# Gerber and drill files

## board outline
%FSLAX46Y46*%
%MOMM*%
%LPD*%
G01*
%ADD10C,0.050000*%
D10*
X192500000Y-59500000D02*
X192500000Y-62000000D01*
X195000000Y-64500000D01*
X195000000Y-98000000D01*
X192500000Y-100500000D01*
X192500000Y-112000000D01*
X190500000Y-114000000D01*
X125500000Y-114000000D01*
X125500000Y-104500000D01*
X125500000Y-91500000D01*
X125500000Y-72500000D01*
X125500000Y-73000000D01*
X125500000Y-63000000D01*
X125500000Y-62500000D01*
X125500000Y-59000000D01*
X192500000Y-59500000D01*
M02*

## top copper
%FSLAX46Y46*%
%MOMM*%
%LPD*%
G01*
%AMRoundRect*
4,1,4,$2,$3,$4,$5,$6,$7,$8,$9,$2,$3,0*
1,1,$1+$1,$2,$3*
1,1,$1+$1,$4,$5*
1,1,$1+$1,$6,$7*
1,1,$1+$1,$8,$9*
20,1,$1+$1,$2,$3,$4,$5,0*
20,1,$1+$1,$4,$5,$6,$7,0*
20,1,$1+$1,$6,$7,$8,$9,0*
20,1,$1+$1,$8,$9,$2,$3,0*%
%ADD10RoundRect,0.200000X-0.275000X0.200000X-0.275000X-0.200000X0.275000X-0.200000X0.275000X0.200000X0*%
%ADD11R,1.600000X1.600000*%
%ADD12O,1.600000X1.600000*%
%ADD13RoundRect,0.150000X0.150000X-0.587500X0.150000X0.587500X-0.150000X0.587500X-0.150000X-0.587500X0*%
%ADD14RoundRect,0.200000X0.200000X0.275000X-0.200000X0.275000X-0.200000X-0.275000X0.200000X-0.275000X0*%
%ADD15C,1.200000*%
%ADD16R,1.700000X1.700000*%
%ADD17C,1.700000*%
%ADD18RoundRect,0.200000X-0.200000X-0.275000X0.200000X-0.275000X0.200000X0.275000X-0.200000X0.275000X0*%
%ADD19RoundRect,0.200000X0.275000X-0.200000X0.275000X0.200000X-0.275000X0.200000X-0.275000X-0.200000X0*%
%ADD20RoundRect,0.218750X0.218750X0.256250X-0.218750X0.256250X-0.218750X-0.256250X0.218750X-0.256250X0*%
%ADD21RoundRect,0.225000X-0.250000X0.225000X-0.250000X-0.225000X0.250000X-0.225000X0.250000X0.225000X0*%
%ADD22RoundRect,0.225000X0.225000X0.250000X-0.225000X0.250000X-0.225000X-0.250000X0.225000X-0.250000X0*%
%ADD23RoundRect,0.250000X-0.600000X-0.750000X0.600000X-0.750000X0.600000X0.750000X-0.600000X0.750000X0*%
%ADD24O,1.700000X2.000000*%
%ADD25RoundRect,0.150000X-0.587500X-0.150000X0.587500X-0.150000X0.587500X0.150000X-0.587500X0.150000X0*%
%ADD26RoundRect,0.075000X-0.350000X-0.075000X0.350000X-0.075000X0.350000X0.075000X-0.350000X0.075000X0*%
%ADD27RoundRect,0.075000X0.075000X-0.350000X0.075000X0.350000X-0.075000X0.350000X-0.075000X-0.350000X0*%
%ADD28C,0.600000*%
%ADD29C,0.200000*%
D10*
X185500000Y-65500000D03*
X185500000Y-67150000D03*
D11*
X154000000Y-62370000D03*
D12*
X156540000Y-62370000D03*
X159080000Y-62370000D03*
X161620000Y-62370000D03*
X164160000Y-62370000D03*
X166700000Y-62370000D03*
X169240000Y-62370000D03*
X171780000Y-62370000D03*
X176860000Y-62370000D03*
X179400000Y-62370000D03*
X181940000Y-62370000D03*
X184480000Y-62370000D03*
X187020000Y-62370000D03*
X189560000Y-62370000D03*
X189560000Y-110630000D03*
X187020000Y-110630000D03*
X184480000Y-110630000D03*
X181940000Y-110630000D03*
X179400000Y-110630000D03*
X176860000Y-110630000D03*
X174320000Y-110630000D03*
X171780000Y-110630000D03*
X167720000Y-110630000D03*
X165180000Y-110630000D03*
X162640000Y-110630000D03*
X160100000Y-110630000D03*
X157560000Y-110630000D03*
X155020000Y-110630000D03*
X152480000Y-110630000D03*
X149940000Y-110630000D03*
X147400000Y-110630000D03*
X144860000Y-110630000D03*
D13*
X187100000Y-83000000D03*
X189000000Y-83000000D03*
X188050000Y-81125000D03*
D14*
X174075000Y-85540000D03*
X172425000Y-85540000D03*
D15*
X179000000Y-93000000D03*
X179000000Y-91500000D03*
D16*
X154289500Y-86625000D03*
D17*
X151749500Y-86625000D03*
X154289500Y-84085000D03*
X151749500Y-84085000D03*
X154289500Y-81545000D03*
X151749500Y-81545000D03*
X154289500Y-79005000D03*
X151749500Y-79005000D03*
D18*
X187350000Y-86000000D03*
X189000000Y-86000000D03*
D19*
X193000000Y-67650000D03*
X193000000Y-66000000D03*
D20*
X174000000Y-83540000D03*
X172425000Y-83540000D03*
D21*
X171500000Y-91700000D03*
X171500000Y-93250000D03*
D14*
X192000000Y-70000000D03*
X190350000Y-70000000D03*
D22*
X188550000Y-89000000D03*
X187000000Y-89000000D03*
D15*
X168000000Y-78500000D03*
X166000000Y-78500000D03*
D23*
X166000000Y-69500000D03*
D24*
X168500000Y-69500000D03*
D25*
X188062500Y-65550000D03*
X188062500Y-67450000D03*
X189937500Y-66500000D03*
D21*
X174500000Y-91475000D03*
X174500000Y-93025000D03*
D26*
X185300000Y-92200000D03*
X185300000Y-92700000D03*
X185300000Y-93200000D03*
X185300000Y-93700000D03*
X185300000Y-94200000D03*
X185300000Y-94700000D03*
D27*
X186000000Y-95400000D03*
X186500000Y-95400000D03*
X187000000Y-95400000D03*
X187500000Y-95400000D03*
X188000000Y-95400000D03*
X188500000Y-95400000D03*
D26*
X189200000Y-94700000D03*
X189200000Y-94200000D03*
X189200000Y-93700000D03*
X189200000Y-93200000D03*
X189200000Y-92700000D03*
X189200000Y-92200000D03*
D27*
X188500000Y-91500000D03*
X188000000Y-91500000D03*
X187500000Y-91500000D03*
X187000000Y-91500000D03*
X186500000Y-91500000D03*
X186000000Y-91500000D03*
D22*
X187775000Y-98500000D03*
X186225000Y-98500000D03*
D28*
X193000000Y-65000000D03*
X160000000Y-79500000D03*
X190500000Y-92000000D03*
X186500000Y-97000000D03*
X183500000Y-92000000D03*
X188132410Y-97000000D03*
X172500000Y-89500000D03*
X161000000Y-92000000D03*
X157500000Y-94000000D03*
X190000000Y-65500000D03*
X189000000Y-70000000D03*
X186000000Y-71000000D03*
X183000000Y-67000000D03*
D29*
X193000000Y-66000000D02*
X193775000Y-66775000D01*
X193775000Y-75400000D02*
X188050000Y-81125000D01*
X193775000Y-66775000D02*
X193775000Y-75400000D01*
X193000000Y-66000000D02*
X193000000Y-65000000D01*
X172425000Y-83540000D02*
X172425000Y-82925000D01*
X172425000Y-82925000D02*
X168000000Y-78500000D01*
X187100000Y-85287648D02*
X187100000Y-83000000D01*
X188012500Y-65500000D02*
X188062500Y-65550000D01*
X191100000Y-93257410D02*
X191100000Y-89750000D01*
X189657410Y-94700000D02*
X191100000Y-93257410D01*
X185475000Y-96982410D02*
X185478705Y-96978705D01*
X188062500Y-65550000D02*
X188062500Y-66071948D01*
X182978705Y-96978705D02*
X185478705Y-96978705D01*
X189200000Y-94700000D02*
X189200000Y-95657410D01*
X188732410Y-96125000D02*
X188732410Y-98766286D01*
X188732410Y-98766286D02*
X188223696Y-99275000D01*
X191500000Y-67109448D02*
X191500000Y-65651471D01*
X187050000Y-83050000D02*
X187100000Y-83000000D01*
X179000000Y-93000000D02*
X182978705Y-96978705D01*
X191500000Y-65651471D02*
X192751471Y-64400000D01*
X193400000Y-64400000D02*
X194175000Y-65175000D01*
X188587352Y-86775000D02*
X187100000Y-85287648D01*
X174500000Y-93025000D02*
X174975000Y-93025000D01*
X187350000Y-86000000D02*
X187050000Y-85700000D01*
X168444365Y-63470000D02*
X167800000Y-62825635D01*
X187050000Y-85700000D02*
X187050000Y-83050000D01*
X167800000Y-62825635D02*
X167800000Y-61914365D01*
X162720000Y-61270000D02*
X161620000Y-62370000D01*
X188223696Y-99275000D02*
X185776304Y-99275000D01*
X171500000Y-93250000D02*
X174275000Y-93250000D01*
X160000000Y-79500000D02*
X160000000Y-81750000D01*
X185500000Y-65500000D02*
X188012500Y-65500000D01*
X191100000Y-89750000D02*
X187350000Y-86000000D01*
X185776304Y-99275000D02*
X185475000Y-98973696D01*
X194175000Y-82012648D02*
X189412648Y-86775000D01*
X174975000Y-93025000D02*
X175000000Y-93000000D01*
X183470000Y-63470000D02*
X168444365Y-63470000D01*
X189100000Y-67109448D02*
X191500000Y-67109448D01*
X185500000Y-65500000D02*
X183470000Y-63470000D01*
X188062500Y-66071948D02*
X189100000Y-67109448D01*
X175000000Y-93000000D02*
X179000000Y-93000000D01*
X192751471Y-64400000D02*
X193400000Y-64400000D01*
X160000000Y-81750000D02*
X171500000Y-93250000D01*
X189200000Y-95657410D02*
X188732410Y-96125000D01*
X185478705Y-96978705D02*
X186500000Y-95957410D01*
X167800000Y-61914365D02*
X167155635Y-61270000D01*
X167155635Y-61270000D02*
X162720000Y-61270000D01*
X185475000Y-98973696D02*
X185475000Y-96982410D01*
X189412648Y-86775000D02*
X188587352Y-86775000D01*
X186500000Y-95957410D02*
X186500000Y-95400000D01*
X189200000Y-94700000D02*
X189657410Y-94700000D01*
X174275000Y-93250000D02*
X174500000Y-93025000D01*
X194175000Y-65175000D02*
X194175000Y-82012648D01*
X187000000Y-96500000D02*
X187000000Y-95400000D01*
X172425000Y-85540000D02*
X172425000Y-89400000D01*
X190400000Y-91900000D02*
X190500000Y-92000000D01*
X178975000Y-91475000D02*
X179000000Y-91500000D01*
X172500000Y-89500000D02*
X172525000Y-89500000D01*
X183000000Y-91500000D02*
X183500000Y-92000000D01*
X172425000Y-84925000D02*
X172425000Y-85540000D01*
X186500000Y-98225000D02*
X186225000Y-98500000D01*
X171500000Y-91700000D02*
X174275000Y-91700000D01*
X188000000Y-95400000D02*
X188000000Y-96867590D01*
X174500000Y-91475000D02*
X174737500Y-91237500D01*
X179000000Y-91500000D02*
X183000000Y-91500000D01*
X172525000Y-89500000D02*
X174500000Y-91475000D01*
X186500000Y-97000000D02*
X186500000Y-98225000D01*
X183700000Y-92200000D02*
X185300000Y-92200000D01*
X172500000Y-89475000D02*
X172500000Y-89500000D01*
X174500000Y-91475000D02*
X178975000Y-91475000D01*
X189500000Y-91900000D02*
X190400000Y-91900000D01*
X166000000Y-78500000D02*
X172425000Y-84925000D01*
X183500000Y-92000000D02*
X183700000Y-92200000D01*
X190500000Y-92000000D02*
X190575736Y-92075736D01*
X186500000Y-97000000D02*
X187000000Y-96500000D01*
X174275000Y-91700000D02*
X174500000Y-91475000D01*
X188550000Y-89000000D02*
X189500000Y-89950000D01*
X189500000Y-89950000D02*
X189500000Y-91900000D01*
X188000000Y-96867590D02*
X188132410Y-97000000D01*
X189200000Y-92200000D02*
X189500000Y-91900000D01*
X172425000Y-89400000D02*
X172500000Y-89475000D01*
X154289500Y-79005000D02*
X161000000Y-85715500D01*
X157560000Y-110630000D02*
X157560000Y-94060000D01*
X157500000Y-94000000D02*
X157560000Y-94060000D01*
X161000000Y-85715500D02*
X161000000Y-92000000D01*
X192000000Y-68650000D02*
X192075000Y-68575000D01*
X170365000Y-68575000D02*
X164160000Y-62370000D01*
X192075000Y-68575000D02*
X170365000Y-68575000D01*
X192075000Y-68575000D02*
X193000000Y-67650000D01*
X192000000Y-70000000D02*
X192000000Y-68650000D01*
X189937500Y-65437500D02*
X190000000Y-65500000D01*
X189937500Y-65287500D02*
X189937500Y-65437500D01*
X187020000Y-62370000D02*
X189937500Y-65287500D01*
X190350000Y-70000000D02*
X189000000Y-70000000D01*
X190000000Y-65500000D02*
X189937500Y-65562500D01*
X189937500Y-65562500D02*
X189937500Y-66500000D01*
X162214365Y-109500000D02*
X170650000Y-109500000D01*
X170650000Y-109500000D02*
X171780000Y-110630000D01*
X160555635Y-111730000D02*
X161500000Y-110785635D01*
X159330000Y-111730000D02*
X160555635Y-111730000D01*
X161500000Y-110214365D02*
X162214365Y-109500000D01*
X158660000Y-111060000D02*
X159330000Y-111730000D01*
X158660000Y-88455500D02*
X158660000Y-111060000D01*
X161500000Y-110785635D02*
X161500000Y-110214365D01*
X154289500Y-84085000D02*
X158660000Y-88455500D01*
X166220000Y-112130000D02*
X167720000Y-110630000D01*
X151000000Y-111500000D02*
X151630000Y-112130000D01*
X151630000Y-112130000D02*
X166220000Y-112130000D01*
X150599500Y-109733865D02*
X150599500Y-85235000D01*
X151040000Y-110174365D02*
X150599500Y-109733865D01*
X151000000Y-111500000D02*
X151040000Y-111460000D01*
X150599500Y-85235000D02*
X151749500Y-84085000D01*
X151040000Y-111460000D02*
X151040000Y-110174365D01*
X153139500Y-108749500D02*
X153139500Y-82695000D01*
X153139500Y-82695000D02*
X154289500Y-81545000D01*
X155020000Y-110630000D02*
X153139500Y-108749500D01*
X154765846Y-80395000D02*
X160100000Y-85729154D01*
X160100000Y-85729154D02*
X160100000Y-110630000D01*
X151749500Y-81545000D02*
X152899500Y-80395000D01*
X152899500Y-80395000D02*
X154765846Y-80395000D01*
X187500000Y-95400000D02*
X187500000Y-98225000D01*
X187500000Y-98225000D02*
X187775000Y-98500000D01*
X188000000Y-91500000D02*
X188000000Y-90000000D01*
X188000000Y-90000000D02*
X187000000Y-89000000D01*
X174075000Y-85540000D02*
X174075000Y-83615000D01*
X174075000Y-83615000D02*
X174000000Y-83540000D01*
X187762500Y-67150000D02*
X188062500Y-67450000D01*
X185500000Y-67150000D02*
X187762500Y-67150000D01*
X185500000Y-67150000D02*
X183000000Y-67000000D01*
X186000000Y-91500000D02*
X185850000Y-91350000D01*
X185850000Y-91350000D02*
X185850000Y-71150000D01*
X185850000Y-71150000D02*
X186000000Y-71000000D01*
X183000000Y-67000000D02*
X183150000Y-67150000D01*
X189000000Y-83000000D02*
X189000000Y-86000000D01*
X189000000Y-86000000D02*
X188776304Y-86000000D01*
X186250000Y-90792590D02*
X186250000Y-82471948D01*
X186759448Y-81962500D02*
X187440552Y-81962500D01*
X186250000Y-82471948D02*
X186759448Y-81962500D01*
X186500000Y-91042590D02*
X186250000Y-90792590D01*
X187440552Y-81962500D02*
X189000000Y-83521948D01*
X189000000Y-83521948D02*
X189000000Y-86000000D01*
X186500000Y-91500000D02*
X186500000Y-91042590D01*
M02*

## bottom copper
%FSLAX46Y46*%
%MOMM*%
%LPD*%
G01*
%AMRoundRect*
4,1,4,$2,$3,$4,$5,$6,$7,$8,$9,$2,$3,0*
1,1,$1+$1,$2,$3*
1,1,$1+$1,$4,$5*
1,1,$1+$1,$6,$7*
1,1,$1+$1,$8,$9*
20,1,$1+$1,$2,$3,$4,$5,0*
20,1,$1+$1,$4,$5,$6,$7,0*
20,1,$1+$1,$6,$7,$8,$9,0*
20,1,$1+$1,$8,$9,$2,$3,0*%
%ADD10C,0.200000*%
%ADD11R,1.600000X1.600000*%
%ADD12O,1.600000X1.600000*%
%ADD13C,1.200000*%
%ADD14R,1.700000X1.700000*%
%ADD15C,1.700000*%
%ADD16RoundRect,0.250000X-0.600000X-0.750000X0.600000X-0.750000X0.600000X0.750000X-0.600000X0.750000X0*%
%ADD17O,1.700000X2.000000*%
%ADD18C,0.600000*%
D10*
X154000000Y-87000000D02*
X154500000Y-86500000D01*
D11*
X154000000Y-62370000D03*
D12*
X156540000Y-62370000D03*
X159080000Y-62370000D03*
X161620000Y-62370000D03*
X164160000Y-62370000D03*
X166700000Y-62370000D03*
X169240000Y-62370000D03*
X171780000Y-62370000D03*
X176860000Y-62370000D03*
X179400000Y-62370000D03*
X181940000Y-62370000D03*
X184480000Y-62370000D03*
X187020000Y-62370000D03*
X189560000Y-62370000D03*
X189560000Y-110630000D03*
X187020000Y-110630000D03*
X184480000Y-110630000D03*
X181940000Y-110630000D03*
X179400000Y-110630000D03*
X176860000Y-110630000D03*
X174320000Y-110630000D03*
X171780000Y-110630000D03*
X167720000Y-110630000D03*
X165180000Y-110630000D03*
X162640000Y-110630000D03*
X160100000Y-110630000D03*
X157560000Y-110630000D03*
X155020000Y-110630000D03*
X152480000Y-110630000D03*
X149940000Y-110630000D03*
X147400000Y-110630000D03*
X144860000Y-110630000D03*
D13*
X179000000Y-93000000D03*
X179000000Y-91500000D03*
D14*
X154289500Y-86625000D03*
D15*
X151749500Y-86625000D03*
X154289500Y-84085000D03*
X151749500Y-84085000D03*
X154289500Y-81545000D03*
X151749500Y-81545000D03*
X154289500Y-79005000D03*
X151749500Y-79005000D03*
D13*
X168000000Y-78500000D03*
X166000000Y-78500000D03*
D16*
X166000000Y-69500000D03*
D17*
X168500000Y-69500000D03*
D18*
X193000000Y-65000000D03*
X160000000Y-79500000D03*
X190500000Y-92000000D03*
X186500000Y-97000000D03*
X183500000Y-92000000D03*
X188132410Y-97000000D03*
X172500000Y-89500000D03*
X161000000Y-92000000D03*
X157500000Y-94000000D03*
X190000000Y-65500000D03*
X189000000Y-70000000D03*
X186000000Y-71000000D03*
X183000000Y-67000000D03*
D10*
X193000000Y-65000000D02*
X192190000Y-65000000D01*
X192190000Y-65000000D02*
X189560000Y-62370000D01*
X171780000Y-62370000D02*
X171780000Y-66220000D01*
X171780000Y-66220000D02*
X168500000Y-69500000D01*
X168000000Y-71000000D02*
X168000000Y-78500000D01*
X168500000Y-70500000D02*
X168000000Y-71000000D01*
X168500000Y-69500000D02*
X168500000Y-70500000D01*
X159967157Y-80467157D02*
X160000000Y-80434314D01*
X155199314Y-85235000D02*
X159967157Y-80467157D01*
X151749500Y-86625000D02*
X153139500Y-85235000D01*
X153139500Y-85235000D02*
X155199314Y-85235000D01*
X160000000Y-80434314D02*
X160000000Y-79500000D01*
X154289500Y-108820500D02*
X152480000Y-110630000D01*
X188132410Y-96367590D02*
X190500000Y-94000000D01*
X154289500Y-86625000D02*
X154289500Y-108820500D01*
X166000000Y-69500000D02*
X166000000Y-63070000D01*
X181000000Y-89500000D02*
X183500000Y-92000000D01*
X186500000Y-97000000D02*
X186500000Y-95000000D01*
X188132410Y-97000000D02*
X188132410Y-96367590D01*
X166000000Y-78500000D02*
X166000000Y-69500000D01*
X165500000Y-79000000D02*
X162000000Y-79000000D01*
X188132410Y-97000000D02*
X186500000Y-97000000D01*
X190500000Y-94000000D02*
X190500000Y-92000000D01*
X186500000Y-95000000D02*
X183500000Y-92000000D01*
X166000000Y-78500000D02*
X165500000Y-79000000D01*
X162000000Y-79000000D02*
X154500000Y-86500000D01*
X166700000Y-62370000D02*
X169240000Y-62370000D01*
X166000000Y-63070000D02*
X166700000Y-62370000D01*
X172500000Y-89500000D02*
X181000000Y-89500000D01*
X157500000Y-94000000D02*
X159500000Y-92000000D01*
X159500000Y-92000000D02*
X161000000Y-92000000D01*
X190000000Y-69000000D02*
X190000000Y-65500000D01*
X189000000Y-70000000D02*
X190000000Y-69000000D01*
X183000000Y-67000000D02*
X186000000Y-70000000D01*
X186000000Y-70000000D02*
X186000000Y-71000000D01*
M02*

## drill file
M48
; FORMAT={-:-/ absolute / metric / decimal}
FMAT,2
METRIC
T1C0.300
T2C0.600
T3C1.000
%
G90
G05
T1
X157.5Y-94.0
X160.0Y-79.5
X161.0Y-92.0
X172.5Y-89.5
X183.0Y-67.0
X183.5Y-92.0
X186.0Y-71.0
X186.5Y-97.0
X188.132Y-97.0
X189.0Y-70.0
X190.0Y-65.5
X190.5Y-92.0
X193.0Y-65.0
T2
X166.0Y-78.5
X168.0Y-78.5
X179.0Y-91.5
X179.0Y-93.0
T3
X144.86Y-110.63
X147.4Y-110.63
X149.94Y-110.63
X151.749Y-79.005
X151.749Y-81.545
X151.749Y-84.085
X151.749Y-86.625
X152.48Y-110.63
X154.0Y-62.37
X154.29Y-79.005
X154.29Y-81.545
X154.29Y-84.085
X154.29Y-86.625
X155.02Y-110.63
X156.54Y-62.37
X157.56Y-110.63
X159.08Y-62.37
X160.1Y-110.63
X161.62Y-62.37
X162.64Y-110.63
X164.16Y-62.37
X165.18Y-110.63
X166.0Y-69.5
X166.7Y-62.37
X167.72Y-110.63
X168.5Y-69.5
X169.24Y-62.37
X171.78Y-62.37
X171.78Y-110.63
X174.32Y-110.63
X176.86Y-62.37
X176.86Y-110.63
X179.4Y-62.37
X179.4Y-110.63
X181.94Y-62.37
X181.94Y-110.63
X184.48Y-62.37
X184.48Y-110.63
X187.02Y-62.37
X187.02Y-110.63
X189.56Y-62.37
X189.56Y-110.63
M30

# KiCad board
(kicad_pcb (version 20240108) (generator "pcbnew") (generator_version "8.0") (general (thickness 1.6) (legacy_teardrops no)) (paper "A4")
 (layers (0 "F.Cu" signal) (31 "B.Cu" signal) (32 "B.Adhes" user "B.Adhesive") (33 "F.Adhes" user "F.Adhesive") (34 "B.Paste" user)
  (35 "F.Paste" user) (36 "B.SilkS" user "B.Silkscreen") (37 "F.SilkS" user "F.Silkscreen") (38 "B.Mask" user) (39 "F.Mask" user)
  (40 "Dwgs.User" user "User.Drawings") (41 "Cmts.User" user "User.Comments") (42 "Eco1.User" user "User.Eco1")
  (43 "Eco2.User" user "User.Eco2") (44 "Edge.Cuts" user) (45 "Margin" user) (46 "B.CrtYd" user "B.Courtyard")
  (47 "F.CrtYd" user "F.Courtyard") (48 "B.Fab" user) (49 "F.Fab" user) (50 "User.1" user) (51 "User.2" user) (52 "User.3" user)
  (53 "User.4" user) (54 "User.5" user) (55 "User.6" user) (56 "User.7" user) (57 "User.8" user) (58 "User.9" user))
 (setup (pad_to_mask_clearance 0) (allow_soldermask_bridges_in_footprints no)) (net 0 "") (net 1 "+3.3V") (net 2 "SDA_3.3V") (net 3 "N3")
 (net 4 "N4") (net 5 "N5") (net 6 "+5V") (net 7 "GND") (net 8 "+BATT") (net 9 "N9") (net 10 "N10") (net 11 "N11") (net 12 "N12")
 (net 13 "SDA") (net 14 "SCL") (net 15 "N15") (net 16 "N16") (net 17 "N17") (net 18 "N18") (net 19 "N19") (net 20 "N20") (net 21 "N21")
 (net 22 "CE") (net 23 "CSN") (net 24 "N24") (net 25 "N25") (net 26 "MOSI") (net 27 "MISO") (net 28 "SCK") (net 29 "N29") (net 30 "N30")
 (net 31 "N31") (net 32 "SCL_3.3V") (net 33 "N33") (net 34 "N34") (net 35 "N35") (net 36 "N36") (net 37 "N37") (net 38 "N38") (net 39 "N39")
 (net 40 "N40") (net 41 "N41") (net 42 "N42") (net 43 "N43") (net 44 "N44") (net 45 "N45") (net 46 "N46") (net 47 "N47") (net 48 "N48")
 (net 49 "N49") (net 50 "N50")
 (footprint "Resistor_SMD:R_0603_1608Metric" (layer "F.Cu") (at 185.5 66.325 -90)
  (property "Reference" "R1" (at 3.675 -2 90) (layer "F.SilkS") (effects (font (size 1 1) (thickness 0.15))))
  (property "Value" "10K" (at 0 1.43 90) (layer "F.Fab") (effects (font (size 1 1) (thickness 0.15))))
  (pad "1" smd roundrect (at -0.825 0 270) (size 0.8 0.95) (layers "F.Cu" "F.Paste" "F.Mask") (roundrect_rratio 0.25) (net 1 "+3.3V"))
  (pad "2" smd roundrect (at 0.825 0 270) (size 0.8 0.95) (layers "F.Cu" "F.Paste" "F.Mask") (roundrect_rratio 0.25) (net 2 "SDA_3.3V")))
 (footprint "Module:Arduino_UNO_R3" (layer "F.Cu") (at 154 62.37)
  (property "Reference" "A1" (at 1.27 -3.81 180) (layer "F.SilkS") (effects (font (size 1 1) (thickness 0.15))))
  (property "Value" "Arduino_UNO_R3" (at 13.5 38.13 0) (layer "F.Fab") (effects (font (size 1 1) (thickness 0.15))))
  (pad "1" thru_hole rect (at 0 0 90) (size 1.6 1.6) (drill 1) (layers "*.Cu" "*.Mask") (remove_unused_layers no) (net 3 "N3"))
  (pad "2" thru_hole oval (at 2.54 0 90) (size 1.6 1.6) (drill 1) (layers "*.Cu" "*.Mask") (remove_unused_layers no) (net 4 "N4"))
  (pad "3" thru_hole oval (at 5.08 0 90) (size 1.6 1.6) (drill 1) (layers "*.Cu" "*.Mask") (remove_unused_layers no) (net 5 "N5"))
  (pad "4" thru_hole oval (at 7.62 0 90) (size 1.6 1.6) (drill 1) (layers "*.Cu" "*.Mask") (remove_unused_layers no) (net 1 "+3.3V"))
  (pad "5" thru_hole oval (at 10.16 0 90) (size 1.6 1.6) (drill 1) (layers "*.Cu" "*.Mask") (remove_unused_layers no) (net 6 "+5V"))
  (pad "6" thru_hole oval (at 12.7 0 90) (size 1.6 1.6) (drill 1) (layers "*.Cu" "*.Mask") (remove_unused_layers no) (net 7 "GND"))
  (pad "7" thru_hole oval (at 15.24 0 90) (size 1.6 1.6) (drill 1) (layers "*.Cu" "*.Mask") (remove_unused_layers no) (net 7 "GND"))
  (pad "8" thru_hole oval (at 17.78 0 90) (size 1.6 1.6) (drill 1) (layers "*.Cu" "*.Mask") (remove_unused_layers no) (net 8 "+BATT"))
  (pad "9" thru_hole oval (at 22.86 0 90) (size 1.6 1.6) (drill 1) (layers "*.Cu" "*.Mask") (remove_unused_layers no) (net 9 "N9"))
  (pad "10" thru_hole oval (at 25.4 0 90) (size 1.6 1.6) (drill 1) (layers "*.Cu" "*.Mask") (remove_unused_layers no) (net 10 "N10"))
  (pad "11" thru_hole oval (at 27.94 0 90) (size 1.6 1.6) (drill 1) (layers "*.Cu" "*.Mask") (remove_unused_layers no) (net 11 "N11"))
  (pad "12" thru_hole oval (at 30.48 0 90) (size 1.6 1.6) (drill 1) (layers "*.Cu" "*.Mask") (remove_unused_layers no) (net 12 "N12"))
  (pad "13" thru_hole oval (at 33.02 0 90) (size 1.6 1.6) (drill 1) (layers "*.Cu" "*.Mask") (remove_unused_layers no) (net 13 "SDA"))
  (pad "14" thru_hole oval (at 35.56 0 90) (size 1.6 1.6) (drill 1) (layers "*.Cu" "*.Mask") (remove_unused_layers no) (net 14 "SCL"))
  (pad "15" thru_hole oval (at 35.56 48.26 90) (size 1.6 1.6) (drill 1) (layers "*.Cu" "*.Mask") (remove_unused_layers no) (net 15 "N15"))
  (pad "16" thru_hole oval (at 33.02 48.26 90) (size 1.6 1.6) (drill 1) (layers "*.Cu" "*.Mask") (remove_unused_layers no) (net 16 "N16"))
  (pad "17" thru_hole oval (at 30.48 48.26 90) (size 1.6 1.6) (drill 1) (layers "*.Cu" "*.Mask") (remove_unused_layers no) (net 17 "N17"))
  (pad "18" thru_hole oval (at 27.94 48.26 90) (size 1.6 1.6) (drill 1) (layers "*.Cu" "*.Mask") (remove_unused_layers no) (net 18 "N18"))
  (pad "19" thru_hole oval (at 25.4 48.26 90) (size 1.6 1.6) (drill 1) (layers "*.Cu" "*.Mask") (remove_unused_layers no) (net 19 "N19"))
  (pad "20" thru_hole oval (at 22.86 48.26 90) (size 1.6 1.6) (drill 1) (layers "*.Cu" "*.Mask") (remove_unused_layers no) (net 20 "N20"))
  (pad "21" thru_hole oval (at 20.32 48.26 90) (size 1.6 1.6) (drill 1) (layers "*.Cu" "*.Mask") (remove_unused_layers no) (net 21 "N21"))
  (pad "22" thru_hole oval (at 17.78 48.26 90) (size 1.6 1.6) (drill 1) (layers "*.Cu" "*.Mask") (remove_unused_layers no) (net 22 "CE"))
  (pad "23" thru_hole oval (at 13.72 48.26 90) (size 1.6 1.6) (drill 1) (layers "*.Cu" "*.Mask") (remove_unused_layers no) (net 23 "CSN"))
  (pad "24" thru_hole oval (at 11.18 48.26 90) (size 1.6 1.6) (drill 1) (layers "*.Cu" "*.Mask") (remove_unused_layers no) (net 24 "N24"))
  (pad "25" thru_hole oval (at 8.64 48.26 90) (size 1.6 1.6) (drill 1) (layers "*.Cu" "*.Mask") (remove_unused_layers no) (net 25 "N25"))
  (pad "26" thru_hole oval (at 6.1 48.26 90) (size 1.6 1.6) (drill 1) (layers "*.Cu" "*.Mask") (remove_unused_layers no) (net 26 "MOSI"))
  (pad "27" thru_hole oval (at 3.56 48.26 90) (size 1.6 1.6) (drill 1) (layers "*.Cu" "*.Mask") (remove_unused_layers no) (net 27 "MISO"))
  (pad "28" thru_hole oval (at 1.02 48.26 90) (size 1.6 1.6) (drill 1) (layers "*.Cu" "*.Mask") (remove_unused_layers no) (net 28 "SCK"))
  (pad "29" thru_hole oval (at -1.52 48.26 90) (size 1.6 1.6) (drill 1) (layers "*.Cu" "*.Mask") (remove_unused_layers no) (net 7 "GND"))
  (pad "30" thru_hole oval (at -4.06 48.26 90) (size 1.6 1.6) (drill 1) (layers "*.Cu" "*.Mask") (remove_unused_layers no) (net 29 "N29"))
  (pad "31" thru_hole oval (at -6.6 48.26 90) (size 1.6 1.6) (drill 1) (layers "*.Cu" "*.Mask") (remove_unused_layers no) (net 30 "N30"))
  (pad "32" thru_hole oval (at -9.14 48.26 90) (size 1.6 1.6) (drill 1) (layers "*.Cu" "*.Mask") (remove_unused_layers no) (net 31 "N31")))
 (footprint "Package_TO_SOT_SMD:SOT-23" (layer "F.Cu") (at 188.05 82.0625 90)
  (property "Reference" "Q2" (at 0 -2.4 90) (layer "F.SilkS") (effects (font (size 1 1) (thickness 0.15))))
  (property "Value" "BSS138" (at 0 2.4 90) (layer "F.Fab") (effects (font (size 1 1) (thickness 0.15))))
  (pad "1" smd roundrect (at -0.9375 -0.95 90) (size 1.475 0.6) (layers "F.Cu" "F.Paste" "F.Mask") (roundrect_rratio 0.25) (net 1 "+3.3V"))
  (pad "2" smd roundrect (at -0.9375 0.95 90) (size 1.475 0.6) (layers "F.Cu" "F.Paste" "F.Mask") (roundrect_rratio 0.25)
   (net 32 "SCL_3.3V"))
  (pad "3" smd roundrect (at 0.9375 0 90) (size 1.475 0.6) (layers "F.Cu" "F.Paste" "F.Mask") (roundrect_rratio 0.25) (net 14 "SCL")))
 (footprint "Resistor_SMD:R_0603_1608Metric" (layer "F.Cu") (at 173.25 85.54 180)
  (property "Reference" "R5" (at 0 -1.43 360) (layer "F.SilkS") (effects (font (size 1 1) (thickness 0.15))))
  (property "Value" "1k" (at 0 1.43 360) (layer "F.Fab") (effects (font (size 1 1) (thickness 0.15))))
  (pad "1" smd roundrect (at -0.825 0 180) (size 0.8 0.95) (layers "F.Cu" "F.Paste" "F.Mask") (roundrect_rratio 0.25) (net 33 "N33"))
  (pad "2" smd roundrect (at 0.825 0 180) (size 0.8 0.95) (layers "F.Cu" "F.Paste" "F.Mask") (roundrect_rratio 0.25) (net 7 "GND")))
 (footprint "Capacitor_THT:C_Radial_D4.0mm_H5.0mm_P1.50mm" (layer "F.Cu") (at 179 93 90)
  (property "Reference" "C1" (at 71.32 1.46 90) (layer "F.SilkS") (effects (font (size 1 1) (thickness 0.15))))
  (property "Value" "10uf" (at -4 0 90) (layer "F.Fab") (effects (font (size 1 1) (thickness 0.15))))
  (pad "1" thru_hole circle (at 0 0 90) (size 1.2 1.2) (drill 0.6) (layers "*.Cu" "*.Mask") (remove_unused_layers no) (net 1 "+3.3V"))
  (pad "2" thru_hole circle (at 1.5 0 90) (size 1.2 1.2) (drill 0.6) (layers "*.Cu" "*.Mask") (remove_unused_layers no) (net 7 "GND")))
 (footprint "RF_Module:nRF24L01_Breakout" (layer "F.Cu") (at 154.2895 86.625 180)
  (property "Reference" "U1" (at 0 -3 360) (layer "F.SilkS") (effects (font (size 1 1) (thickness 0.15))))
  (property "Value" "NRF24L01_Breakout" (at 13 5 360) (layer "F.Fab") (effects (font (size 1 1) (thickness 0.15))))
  (pad "1" thru_hole rect (at 0 0 180) (size 1.7 1.7) (drill 1) (layers "*.Cu" "*.Mask") (remove_unused_layers no) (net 7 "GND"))
  (pad "2" thru_hole circle (at 2.54 0 180) (size 1.7 1.7) (drill 1) (layers "*.Cu" "*.Mask") (remove_unused_layers no) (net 1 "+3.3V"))
  (pad "3" thru_hole circle (at 0 2.54 180) (size 1.7 1.7) (drill 1) (layers "*.Cu" "*.Mask") (remove_unused_layers no) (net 22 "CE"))
  (pad "4" thru_hole circle (at 2.54 2.54 180) (size 1.7 1.7) (drill 1) (layers "*.Cu" "*.Mask") (remove_unused_layers no) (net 23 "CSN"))
  (pad "5" thru_hole circle (at 0 5.08 180) (size 1.7 1.7) (drill 1) (layers "*.Cu" "*.Mask") (remove_unused_layers no) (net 28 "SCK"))
  (pad "6" thru_hole circle (at 2.54 5.08 180) (size 1.7 1.7) (drill 1) (layers "*.Cu" "*.Mask") (remove_unused_layers no) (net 26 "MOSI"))
  (pad "7" thru_hole circle (at 0 7.62 180) (size 1.7 1.7) (drill 1) (layers "*.Cu" "*.Mask") (remove_unused_layers no) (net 27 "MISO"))
  (pad "8" thru_hole circle (at 2.54 7.62 180) (size 1.7 1.7) (drill 1) (layers "*.Cu" "*.Mask") (remove_unused_layers no) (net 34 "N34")))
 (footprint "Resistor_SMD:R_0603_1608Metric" (layer "F.Cu") (at 188.175 86)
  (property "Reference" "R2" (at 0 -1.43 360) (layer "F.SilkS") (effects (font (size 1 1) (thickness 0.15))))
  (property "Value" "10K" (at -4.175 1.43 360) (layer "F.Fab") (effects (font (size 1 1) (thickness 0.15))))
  (pad "1" smd roundrect (at -0.825 0) (size 0.8 0.95) (layers "F.Cu" "F.Paste" "F.Mask") (roundrect_rratio 0.25) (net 1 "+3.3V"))
  (pad "2" smd roundrect (at 0.825 0) (size 0.8 0.95) (layers "F.Cu" "F.Paste" "F.Mask") (roundrect_rratio 0.25) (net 32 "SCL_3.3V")))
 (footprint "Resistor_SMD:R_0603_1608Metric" (layer "F.Cu") (at 193 66.825 90)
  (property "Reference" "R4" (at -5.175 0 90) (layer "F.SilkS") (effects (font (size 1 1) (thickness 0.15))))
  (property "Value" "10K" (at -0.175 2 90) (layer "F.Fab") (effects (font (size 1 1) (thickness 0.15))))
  (pad "1" smd roundrect (at -0.825 0 90) (size 0.8 0.95) (layers "F.Cu" "F.Paste" "F.Mask") (roundrect_rratio 0.25) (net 6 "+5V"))
  (pad "2" smd roundrect (at 0.825 0 90) (size 0.8 0.95) (layers "F.Cu" "F.Paste" "F.Mask") (roundrect_rratio 0.25) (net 14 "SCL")))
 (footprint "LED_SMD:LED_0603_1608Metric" (layer "F.Cu") (at 173.2125 83.54 180)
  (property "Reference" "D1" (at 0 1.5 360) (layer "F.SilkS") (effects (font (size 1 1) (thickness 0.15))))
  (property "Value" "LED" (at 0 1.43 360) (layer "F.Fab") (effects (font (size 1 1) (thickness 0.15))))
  (pad "1" smd roundrect (at -0.7875 0 180) (size 0.875 0.95) (layers "F.Cu" "F.Paste" "F.Mask") (roundrect_rratio 0.25) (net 33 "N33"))
  (pad "2" smd roundrect (at 0.7875 0 180) (size 0.875 0.95) (layers "F.Cu" "F.Paste" "F.Mask") (roundrect_rratio 0.25) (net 8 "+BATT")))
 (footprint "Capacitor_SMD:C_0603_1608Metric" (layer "F.Cu") (at 171.5 92.475 -90)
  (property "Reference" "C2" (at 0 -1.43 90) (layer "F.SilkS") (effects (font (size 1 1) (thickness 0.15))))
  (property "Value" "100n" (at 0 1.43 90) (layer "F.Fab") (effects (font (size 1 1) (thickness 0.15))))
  (pad "1" smd roundrect (at -0.775 0 270) (size 0.9 0.95) (layers "F.Cu" "F.Paste" "F.Mask") (roundrect_rratio 0.25) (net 7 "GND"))
  (pad "2" smd roundrect (at 0.775 0 270) (size 0.9 0.95) (layers "F.Cu" "F.Paste" "F.Mask") (roundrect_rratio 0.25) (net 1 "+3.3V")))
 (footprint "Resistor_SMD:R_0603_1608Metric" (layer "F.Cu") (at 191.175 70 180)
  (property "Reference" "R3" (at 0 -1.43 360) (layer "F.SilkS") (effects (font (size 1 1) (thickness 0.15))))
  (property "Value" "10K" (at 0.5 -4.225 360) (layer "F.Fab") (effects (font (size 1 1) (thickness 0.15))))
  (pad "1" smd roundrect (at -0.825 0 180) (size 0.8 0.95) (layers "F.Cu" "F.Paste" "F.Mask") (roundrect_rratio 0.25) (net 6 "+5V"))
  (pad "2" smd roundrect (at 0.825 0 180) (size 0.8 0.95) (layers "F.Cu" "F.Paste" "F.Mask") (roundrect_rratio 0.25) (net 13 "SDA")))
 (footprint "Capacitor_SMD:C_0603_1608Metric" (layer "F.Cu") (at 187.775 89 180)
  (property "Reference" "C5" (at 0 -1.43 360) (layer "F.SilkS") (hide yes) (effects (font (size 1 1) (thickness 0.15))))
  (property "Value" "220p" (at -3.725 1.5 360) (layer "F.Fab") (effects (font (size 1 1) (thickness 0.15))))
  (pad "1" smd roundrect (at -0.775 0 180) (size 0.9 0.95) (layers "F.Cu" "F.Paste" "F.Mask") (roundrect_rratio 0.25) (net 7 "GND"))
  (pad "2" smd roundrect (at 0.775 0 180) (size 0.9 0.95) (layers "F.Cu" "F.Paste" "F.Mask") (roundrect_rratio 0.25) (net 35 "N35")))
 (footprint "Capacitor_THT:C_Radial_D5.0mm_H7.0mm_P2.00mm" (layer "F.Cu") (at 168 78.5 180)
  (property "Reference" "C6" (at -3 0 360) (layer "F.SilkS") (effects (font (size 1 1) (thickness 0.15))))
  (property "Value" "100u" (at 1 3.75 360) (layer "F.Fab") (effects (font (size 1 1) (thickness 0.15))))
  (pad "1" thru_hole circle (at 0 0 180) (size 1.2 1.2) (drill 0.6) (layers "*.Cu" "*.Mask") (remove_unused_layers no) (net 8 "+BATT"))
  (pad "2" thru_hole circle (at 2 0 180) (size 1.2 1.2) (drill 0.6) (layers "*.Cu" "*.Mask") (remove_unused_layers no) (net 7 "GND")))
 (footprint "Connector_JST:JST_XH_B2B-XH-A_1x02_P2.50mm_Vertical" (layer "F.Cu") (at 166 69.5)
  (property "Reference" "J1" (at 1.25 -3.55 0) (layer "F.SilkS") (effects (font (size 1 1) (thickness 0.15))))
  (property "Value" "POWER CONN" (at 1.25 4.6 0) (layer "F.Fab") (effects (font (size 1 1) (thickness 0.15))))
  (pad "1" thru_hole roundrect (at 0 0) (size 1.7 2) (drill 1) (layers "*.Cu" "*.Mask") (remove_unused_layers no)
   (roundrect_rratio 0.147059) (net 7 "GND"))
  (pad "2" thru_hole oval (at 2.5 0) (size 1.7 2) (drill 1) (layers "*.Cu" "*.Mask") (remove_unused_layers no) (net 8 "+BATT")))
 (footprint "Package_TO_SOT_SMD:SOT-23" (layer "F.Cu") (at 189 66.5)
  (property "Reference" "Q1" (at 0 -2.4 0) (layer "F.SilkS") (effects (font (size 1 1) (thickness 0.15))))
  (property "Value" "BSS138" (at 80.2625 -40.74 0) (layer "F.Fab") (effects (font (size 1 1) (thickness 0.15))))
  (pad "1" smd roundrect (at -0.9375 -0.95) (size 1.475 0.6) (layers "F.Cu" "F.Paste" "F.Mask") (roundrect_rratio 0.25) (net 1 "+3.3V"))
  (pad "2" smd roundrect (at -0.9375 0.95) (size 1.475 0.6) (layers "F.Cu" "F.Paste" "F.Mask") (roundrect_rratio 0.25) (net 2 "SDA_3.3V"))
  (pad "3" smd roundrect (at 0.9375 0) (size 1.475 0.6) (layers "F.Cu" "F.Paste" "F.Mask") (roundrect_rratio 0.25) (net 13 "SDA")))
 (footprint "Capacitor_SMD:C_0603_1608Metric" (layer "F.Cu") (at 174.5 92.25 -90)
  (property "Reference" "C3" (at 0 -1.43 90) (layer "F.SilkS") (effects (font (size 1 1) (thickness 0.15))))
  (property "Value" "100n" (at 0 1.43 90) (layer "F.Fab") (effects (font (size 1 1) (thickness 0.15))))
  (pad "1" smd roundrect (at -0.775 0 270) (size 0.9 0.95) (layers "F.Cu" "F.Paste" "F.Mask") (roundrect_rratio 0.25) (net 7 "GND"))
  (pad "2" smd roundrect (at 0.775 0 270) (size 0.9 0.95) (layers "F.Cu" "F.Paste" "F.Mask") (roundrect_rratio 0.25) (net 1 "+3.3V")))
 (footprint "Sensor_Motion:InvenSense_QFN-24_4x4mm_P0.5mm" (layer "F.Cu") (at 187.25 93.45)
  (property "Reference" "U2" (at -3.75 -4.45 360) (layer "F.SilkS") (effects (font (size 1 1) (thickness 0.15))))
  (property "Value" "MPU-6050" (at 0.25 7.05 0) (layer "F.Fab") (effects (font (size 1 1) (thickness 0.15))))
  (pad "1" smd roundrect (at -1.95 -1.25) (size 0.85 0.3) (layers "F.Cu" "F.Paste" "F.Mask") (roundrect_rratio 0.25) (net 7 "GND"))
  (pad "2" smd roundrect (at -1.95 -0.75) (size 0.85 0.3) (layers "F.Cu" "F.Paste" "F.Mask") (roundrect_rratio 0.25) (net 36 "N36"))
  (pad "3" smd roundrect (at -1.95 -0.25) (size 0.85 0.3) (layers "F.Cu" "F.Paste" "F.Mask") (roundrect_rratio 0.25) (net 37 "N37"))
  (pad "4" smd roundrect (at -1.95 0.25) (size 0.85 0.3) (layers "F.Cu" "F.Paste" "F.Mask") (roundrect_rratio 0.25) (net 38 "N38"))
  (pad "5" smd roundrect (at -1.95 0.75) (size 0.85 0.3) (layers "F.Cu" "F.Paste" "F.Mask") (roundrect_rratio 0.25) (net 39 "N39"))
  (pad "6" smd roundrect (at -1.95 1.25) (size 0.85 0.3) (layers "F.Cu" "F.Paste" "F.Mask") (roundrect_rratio 0.25) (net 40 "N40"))
  (pad "7" smd roundrect (at -1.25 1.95 90) (size 0.85 0.3) (layers "F.Cu" "F.Paste" "F.Mask") (roundrect_rratio 0.25) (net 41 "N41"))
  (pad "8" smd roundrect (at -0.75 1.95 90) (size 0.85 0.3) (layers "F.Cu" "F.Paste" "F.Mask") (roundrect_rratio 0.25) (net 1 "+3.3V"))
  (pad "9" smd roundrect (at -0.25 1.95 90) (size 0.85 0.3) (layers "F.Cu" "F.Paste" "F.Mask") (roundrect_rratio 0.25) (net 7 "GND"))
  (pad "10" smd roundrect (at 0.25 1.95 90) (size 0.85 0.3) (layers "F.Cu" "F.Paste" "F.Mask") (roundrect_rratio 0.25) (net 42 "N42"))
  (pad "11" smd roundrect (at 0.75 1.95 90) (size 0.85 0.3) (layers "F.Cu" "F.Paste" "F.Mask") (roundrect_rratio 0.25) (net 7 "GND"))
  (pad "12" smd roundrect (at 1.25 1.95 90) (size 0.85 0.3) (layers "F.Cu" "F.Paste" "F.Mask") (roundrect_rratio 0.25) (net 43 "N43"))
  (pad "13" smd roundrect (at 1.95 1.25) (size 0.85 0.3) (layers "F.Cu" "F.Paste" "F.Mask") (roundrect_rratio 0.25) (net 1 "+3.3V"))
  (pad "14" smd roundrect (at 1.95 0.75) (size 0.85 0.3) (layers "F.Cu" "F.Paste" "F.Mask") (roundrect_rratio 0.25) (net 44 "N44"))
  (pad "15" smd roundrect (at 1.95 0.25) (size 0.85 0.3) (layers "F.Cu" "F.Paste" "F.Mask") (roundrect_rratio 0.25) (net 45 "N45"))
  (pad "16" smd roundrect (at 1.95 -0.25) (size 0.85 0.3) (layers "F.Cu" "F.Paste" "F.Mask") (roundrect_rratio 0.25) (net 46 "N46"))
  (pad "17" smd roundrect (at 1.95 -0.75) (size 0.85 0.3) (layers "F.Cu" "F.Paste" "F.Mask") (roundrect_rratio 0.25) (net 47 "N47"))
  (pad "18" smd roundrect (at 1.95 -1.25) (size 0.85 0.3) (layers "F.Cu" "F.Paste" "F.Mask") (roundrect_rratio 0.25) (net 7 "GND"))
  (pad "19" smd roundrect (at 1.25 -1.95 90) (size 0.85 0.3) (layers "F.Cu" "F.Paste" "F.Mask") (roundrect_rratio 0.25) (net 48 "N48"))
  (pad "20" smd roundrect (at 0.75 -1.95 90) (size 0.85 0.3) (layers "F.Cu" "F.Paste" "F.Mask") (roundrect_rratio 0.25) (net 35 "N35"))
  (pad "21" smd roundrect (at 0.25 -1.95 90) (size 0.85 0.3) (layers "F.Cu" "F.Paste" "F.Mask") (roundrect_rratio 0.25) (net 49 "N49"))
  (pad "22" smd roundrect (at -0.25 -1.95 90) (size 0.85 0.3) (layers "F.Cu" "F.Paste" "F.Mask") (roundrect_rratio 0.25) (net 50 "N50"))
  (pad "23" smd roundrect (at -0.75 -1.95 90) (size 0.85 0.3) (layers "F.Cu" "F.Paste" "F.Mask") (roundrect_rratio 0.25) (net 32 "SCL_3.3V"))
  (pad "24" smd roundrect (at -1.25 -1.95 90) (size 0.85 0.3) (layers "F.Cu" "F.Paste" "F.Mask") (roundrect_rratio 0.25) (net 2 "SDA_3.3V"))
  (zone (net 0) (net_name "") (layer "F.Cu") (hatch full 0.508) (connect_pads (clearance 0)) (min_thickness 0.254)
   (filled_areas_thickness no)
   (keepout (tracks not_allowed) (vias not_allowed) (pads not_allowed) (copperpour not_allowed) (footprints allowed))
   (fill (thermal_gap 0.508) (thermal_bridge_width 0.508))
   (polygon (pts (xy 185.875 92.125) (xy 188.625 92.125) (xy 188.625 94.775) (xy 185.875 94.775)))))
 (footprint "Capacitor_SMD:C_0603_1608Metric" (layer "F.Cu") (at 187 98.5 180)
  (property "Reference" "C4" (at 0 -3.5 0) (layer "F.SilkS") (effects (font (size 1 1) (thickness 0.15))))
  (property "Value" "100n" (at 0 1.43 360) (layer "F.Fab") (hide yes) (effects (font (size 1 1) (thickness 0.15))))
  (pad "1" smd roundrect (at -0.775 0 180) (size 0.9 0.95) (layers "F.Cu" "F.Paste" "F.Mask") (roundrect_rratio 0.25) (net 42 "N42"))
  (pad "2" smd roundrect (at 0.775 0 180) (size 0.9 0.95) (layers "F.Cu" "F.Paste" "F.Mask") (roundrect_rratio 0.25) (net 7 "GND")))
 (gr_line (start 154 87) (end 154.5 86.5) (stroke (width 0.2) (type default)) (layer "B.Cu") (net 7))
 (gr_poly
  (pts (xy 192.5 59.5) (xy 192.5 62) (xy 195 64.5) (xy 195 98) (xy 192.5 100.5) (xy 192.5 112) (xy 190.5 114) (xy 125.5 114)
   (xy 125.5 104.5) (xy 125.5 104.5) (xy 125.5 91.5) (xy 125.5 91.5) (xy 125.5 72.5) (xy 125.5 73) (xy 125.5 63) (xy 125.5 62.5)
   (xy 125.5 59))
  (stroke (width 0.05) (type solid)) (fill none) (layer "Edge.Cuts"))
 (segment (start 193 66) (end 193.775 66.775) (width 0.2) (layer "F.Cu") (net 14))
 (segment (start 193.775 75.4) (end 188.05 81.125) (width 0.2) (layer "F.Cu") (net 14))
 (segment (start 193.775 66.775) (end 193.775 75.4) (width 0.2) (layer "F.Cu") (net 14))
 (segment (start 193 66) (end 193 65) (width 0.2) (layer "F.Cu") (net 14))
 (via (at 193 65) (size 0.6) (drill 0.3) (layers "F.Cu" "B.Cu") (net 14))
 (segment (start 193 65) (end 192.19 65) (width 0.2) (layer "B.Cu") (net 14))
 (segment (start 192.19 65) (end 189.56 62.37) (width 0.2) (layer "B.Cu") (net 14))
 (segment (start 172.425 83.54) (end 172.425 82.925) (width 0.2) (layer "F.Cu") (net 8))
 (segment (start 172.425 82.925) (end 168 78.5) (width 0.2) (layer "F.Cu") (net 8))
 (segment (start 171.78 62.37) (end 171.78 66.22) (width 0.2) (layer "B.Cu") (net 8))
 (segment (start 171.78 66.22) (end 168.5 69.5) (width 0.2) (layer "B.Cu") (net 8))
 (segment (start 168 71) (end 168 78.5) (width 0.2) (layer "B.Cu") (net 8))
 (segment (start 168.5 70.5) (end 168 71) (width 0.2) (layer "B.Cu") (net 8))
 (segment (start 168.5 69.5) (end 168.5 70.5) (width 0.2) (layer "B.Cu") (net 8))
 (segment (start 187.1 85.287648) (end 187.1 83) (width 0.2) (layer "F.Cu") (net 1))
 (segment (start 188.0125 65.5) (end 188.0625 65.55) (width 0.2) (layer "F.Cu") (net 1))
 (segment (start 191.1 93.25741) (end 191.1 89.75) (width 0.2) (layer "F.Cu") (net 1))
 (segment (start 189.65741 94.7) (end 191.1 93.25741) (width 0.2) (layer "F.Cu") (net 1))
 (segment (start 185.475 96.98241) (end 185.478705 96.978705) (width 0.2) (layer "F.Cu") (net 1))
 (segment (start 188.0625 65.55) (end 188.0625 66.071948) (width 0.2) (layer "F.Cu") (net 1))
 (segment (start 182.978705 96.978705) (end 185.478705 96.978705) (width 0.2) (layer "F.Cu") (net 1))
 (segment (start 189.2 94.7) (end 189.2 95.65741) (width 0.2) (layer "F.Cu") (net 1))
 (segment (start 188.73241 96.125) (end 188.73241 98.766286) (width 0.2) (layer "F.Cu") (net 1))
 (segment (start 188.73241 98.766286) (end 188.223696 99.275) (width 0.2) (layer "F.Cu") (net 1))
 (segment (start 191.5 67.109448) (end 191.5 65.651471) (width 0.2) (layer "F.Cu") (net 1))
 (segment (start 187.05 83.05) (end 187.1 83) (width 0.2) (layer "F.Cu") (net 1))
 (segment (start 179 93) (end 182.978705 96.978705) (width 0.2) (layer "F.Cu") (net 1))
 (segment (start 191.5 65.651471) (end 192.751471 64.4) (width 0.2) (layer "F.Cu") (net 1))
 (segment (start 193.4 64.4) (end 194.175 65.175) (width 0.2) (layer "F.Cu") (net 1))
 (segment (start 188.587352 86.775) (end 187.1 85.287648) (width 0.2) (layer "F.Cu") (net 1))
 (segment (start 174.5 93.025) (end 174.975 93.025) (width 0.2) (layer "F.Cu") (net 1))
 (segment (start 187.35 86) (end 187.05 85.7) (width 0.2) (layer "F.Cu") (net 1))
 (segment (start 168.444365 63.47) (end 167.8 62.825635) (width 0.2) (layer "F.Cu") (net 1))
 (segment (start 187.05 85.7) (end 187.05 83.05) (width 0.2) (layer "F.Cu") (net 1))
 (segment (start 167.8 62.825635) (end 167.8 61.914365) (width 0.2) (layer "F.Cu") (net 1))
 (segment (start 162.72 61.27) (end 161.62 62.37) (width 0.2) (layer "F.Cu") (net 1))
 (segment (start 188.223696 99.275) (end 185.776304 99.275) (width 0.2) (layer "F.Cu") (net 1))
 (segment (start 171.5 93.25) (end 174.275 93.25) (width 0.2) (layer "F.Cu") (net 1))
 (segment (start 160 79.5) (end 160 81.75) (width 0.2) (layer "F.Cu") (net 1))
 (segment (start 185.5 65.5) (end 188.0125 65.5) (width 0.2) (layer "F.Cu") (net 1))
 (segment (start 191.1 89.75) (end 187.35 86) (width 0.2) (layer "F.Cu") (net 1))
 (segment (start 185.776304 99.275) (end 185.475 98.973696) (width 0.2) (layer "F.Cu") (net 1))
 (segment (start 194.175 82.012648) (end 189.412648 86.775) (width 0.2) (layer "F.Cu") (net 1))
 (segment (start 174.975 93.025) (end 175 93) (width 0.2) (layer "F.Cu") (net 1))
 (segment (start 183.47 63.47) (end 168.444365 63.47) (width 0.2) (layer "F.Cu") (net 1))
 (segment (start 189.1 67.109448) (end 191.5 67.109448) (width 0.2) (layer "F.Cu") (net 1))
 (segment (start 185.5 65.5) (end 183.47 63.47) (width 0.2) (layer "F.Cu") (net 1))
 (segment (start 188.0625 66.071948) (end 189.1 67.109448) (width 0.2) (layer "F.Cu") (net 1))
 (segment (start 175 93) (end 179 93) (width 0.2) (layer "F.Cu") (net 1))
 (segment (start 192.751471 64.4) (end 193.4 64.4) (width 0.2) (layer "F.Cu") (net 1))
 (segment (start 160 81.75) (end 171.5 93.25) (width 0.2) (layer "F.Cu") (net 1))
 (segment (start 189.2 95.65741) (end 188.73241 96.125) (width 0.2) (layer "F.Cu") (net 1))
 (segment (start 185.478705 96.978705) (end 186.5 95.95741) (width 0.2) (layer "F.Cu") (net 1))
 (segment (start 167.8 61.914365) (end 167.155635 61.27) (width 0.2) (layer "F.Cu") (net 1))
 (segment (start 167.155635 61.27) (end 162.72 61.27) (width 0.2) (layer "F.Cu") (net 1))
 (segment (start 185.475 98.973696) (end 185.475 96.98241) (width 0.2) (layer "F.Cu") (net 1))
 (segment (start 189.412648 86.775) (end 188.587352 86.775) (width 0.2) (layer "F.Cu") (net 1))
 (segment (start 186.5 95.95741) (end 186.5 95.4) (width 0.2) (layer "F.Cu") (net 1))
 (segment (start 189.2 94.7) (end 189.65741 94.7) (width 0.2) (layer "F.Cu") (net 1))
 (segment (start 174.275 93.25) (end 174.5 93.025) (width 0.2) (layer "F.Cu") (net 1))
 (segment (start 194.175 65.175) (end 194.175 82.012648) (width 0.2) (layer "F.Cu") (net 1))
 (via (at 160 79.5) (size 0.6) (drill 0.3) (layers "F.Cu" "B.Cu") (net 1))
 (segment (start 159.967157 80.467157) (end 160 80.434314) (width 0.2) (layer "B.Cu") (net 1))
 (segment (start 155.199314 85.235) (end 159.967157 80.467157) (width 0.2) (layer "B.Cu") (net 1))
 (segment (start 151.7495 86.625) (end 153.1395 85.235) (width 0.2) (layer "B.Cu") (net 1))
 (segment (start 153.1395 85.235) (end 155.199314 85.235) (width 0.2) (layer "B.Cu") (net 1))
 (segment (start 160 80.434314) (end 160 79.5) (width 0.2) (layer "B.Cu") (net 1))
 (segment (start 187 96.5) (end 187 95.4) (width 0.2) (layer "F.Cu") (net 7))
 (segment (start 172.425 85.54) (end 172.425 89.4) (width 0.2) (layer "F.Cu") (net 7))
 (segment (start 190.4 91.9) (end 190.5 92) (width 0.2) (layer "F.Cu") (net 7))
 (segment (start 178.975 91.475) (end 179 91.5) (width 0.2) (layer "F.Cu") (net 7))
 (segment (start 172.5 89.5) (end 172.525 89.5) (width 0.2) (layer "F.Cu") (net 7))
 (segment (start 183 91.5) (end 183.5 92) (width 0.2) (layer "F.Cu") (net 7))
 (segment (start 172.425 84.925) (end 172.425 85.54) (width 0.2) (layer "F.Cu") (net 7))
 (segment (start 186.5 98.225) (end 186.225 98.5) (width 0.2) (layer "F.Cu") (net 7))
 (segment (start 171.5 91.7) (end 174.275 91.7) (width 0.2) (layer "F.Cu") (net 7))
 (segment (start 188 95.4) (end 188 96.86759) (width 0.2) (layer "F.Cu") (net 7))
 (segment (start 174.5 91.475) (end 174.7375 91.2375) (width 0.2) (layer "F.Cu") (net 7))
 (segment (start 179 91.5) (end 183 91.5) (width 0.2) (layer "F.Cu") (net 7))
 (segment (start 172.525 89.5) (end 174.5 91.475) (width 0.2) (layer "F.Cu") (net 7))
 (segment (start 186.5 97) (end 186.5 98.225) (width 0.2) (layer "F.Cu") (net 7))
 (segment (start 183.7 92.2) (end 185.3 92.2) (width 0.2) (layer "F.Cu") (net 7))
 (segment (start 172.5 89.475) (end 172.5 89.5) (width 0.2) (layer "F.Cu") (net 7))
 (segment (start 174.5 91.475) (end 178.975 91.475) (width 0.2) (layer "F.Cu") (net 7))
 (segment (start 189.5 91.9) (end 190.4 91.9) (width 0.2) (layer "F.Cu") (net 7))
 (segment (start 166 78.5) (end 172.425 84.925) (width 0.2) (layer "F.Cu") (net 7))
 (segment (start 183.5 92) (end 183.7 92.2) (width 0.2) (layer "F.Cu") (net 7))
 (segment (start 190.5 92) (end 190.575736 92.075736) (width 0.2) (layer "F.Cu") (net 7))
 (segment (start 186.5 97) (end 187 96.5) (width 0.2) (layer "F.Cu") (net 7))
 (segment (start 174.275 91.7) (end 174.5 91.475) (width 0.2) (layer "F.Cu") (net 7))
 (segment (start 188.55 89) (end 189.5 89.95) (width 0.2) (layer "F.Cu") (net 7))
 (segment (start 189.5 89.95) (end 189.5 91.9) (width 0.2) (layer "F.Cu") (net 7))
 (segment (start 188 96.86759) (end 188.13241 97) (width 0.2) (layer "F.Cu") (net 7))
 (segment (start 189.2 92.2) (end 189.5 91.9) (width 0.2) (layer "F.Cu") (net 7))
 (segment (start 172.425 89.4) (end 172.5 89.475) (width 0.2) (layer "F.Cu") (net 7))
 (via (at 190.5 92) (size 0.6) (drill 0.3) (layers "F.Cu" "B.Cu") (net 7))
 (via (at 186.5 97) (size 0.6) (drill 0.3) (layers "F.Cu" "B.Cu") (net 7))
 (via (at 183.5 92) (size 0.6) (drill 0.3) (layers "F.Cu" "B.Cu") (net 7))
 (via (at 188.13241 97) (size 0.6) (drill 0.3) (layers "F.Cu" "B.Cu") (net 7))
 (via (at 172.5 89.5) (size 0.6) (drill 0.3) (layers "F.Cu" "B.Cu") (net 7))
 (segment (start 154.2895 108.8205) (end 152.48 110.63) (width 0.2) (layer "B.Cu") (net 7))
 (segment (start 188.13241 96.36759) (end 190.5 94) (width 0.2) (layer "B.Cu") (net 7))
 (segment (start 154.2895 86.625) (end 154.2895 108.8205) (width 0.2) (layer "B.Cu") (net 7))
 (segment (start 166 69.5) (end 166 63.07) (width 0.2) (layer "B.Cu") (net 7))
 (segment (start 181 89.5) (end 183.5 92) (width 0.2) (layer "B.Cu") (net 7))
 (segment (start 186.5 97) (end 186.5 95) (width 0.2) (layer "B.Cu") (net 7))
 (segment (start 188.13241 97) (end 188.13241 96.36759) (width 0.2) (layer "B.Cu") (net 7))
 (segment (start 166 78.5) (end 166 69.5) (width 0.2) (layer "B.Cu") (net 7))
 (segment (start 165.5 79) (end 162 79) (width 0.2) (layer "B.Cu") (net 7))
 (segment (start 188.13241 97) (end 186.5 97) (width 0.2) (layer "B.Cu") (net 7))
 (segment (start 190.5 94) (end 190.5 92) (width 0.2) (layer "B.Cu") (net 7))
 (segment (start 186.5 95) (end 183.5 92) (width 0.2) (layer "B.Cu") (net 7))
 (segment (start 166 78.5) (end 165.5 79) (width 0.2) (layer "B.Cu") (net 7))
 (segment (start 162 79) (end 154.5 86.5) (width 0.2) (layer "B.Cu") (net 7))
 (segment (start 166.7 62.37) (end 169.24 62.37) (width 0.2) (layer "B.Cu") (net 7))
 (segment (start 166 63.07) (end 166.7 62.37) (width 0.2) (layer "B.Cu") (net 7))
 (segment (start 172.5 89.5) (end 181 89.5) (width 0.2) (layer "B.Cu") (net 7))
 (segment (start 154.2895 79.005) (end 161 85.7155) (width 0.2) (layer "F.Cu") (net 27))
 (segment (start 157.56 110.63) (end 157.56 94.06) (width 0.2) (layer "F.Cu") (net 27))
 (segment (start 157.5 94) (end 157.56 94.06) (width 0.2) (layer "F.Cu") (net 27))
 (segment (start 161 85.7155) (end 161 92) (width 0.2) (layer "F.Cu") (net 27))
 (via (at 161 92) (size 0.6) (drill 0.3) (layers "F.Cu" "B.Cu") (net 27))
 (via (at 157.5 94) (size 0.6) (drill 0.3) (layers "F.Cu" "B.Cu") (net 27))
 (segment (start 157.5 94) (end 159.5 92) (width 0.2) (layer "B.Cu") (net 27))
 (segment (start 159.5 92) (end 161 92) (width 0.2) (layer "B.Cu") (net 27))
 (segment (start 192 68.65) (end 192.075 68.575) (width 0.2) (layer "F.Cu") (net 6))
 (segment (start 170.365 68.575) (end 164.16 62.37) (width 0.2) (layer "F.Cu") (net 6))
 (segment (start 192.075 68.575) (end 170.365 68.575) (width 0.2) (layer "F.Cu") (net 6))
 (segment (start 192.075 68.575) (end 193 67.65) (width 0.2) (layer "F.Cu") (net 6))
 (segment (start 192 70) (end 192 68.65) (width 0.2) (layer "F.Cu") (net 6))
 (segment (start 189.9375 65.4375) (end 190 65.5) (width 0.2) (layer "F.Cu") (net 13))
 (segment (start 189.9375 65.2875) (end 189.9375 65.4375) (width 0.2) (layer "F.Cu") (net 13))
 (segment (start 187.02 62.37) (end 189.9375 65.2875) (width 0.2) (layer "F.Cu") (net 13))
 (segment (start 190.35 70) (end 189 70) (width 0.2) (layer "F.Cu") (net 13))
 (segment (start 190 65.5) (end 189.9375 65.5625) (width 0.2) (layer "F.Cu") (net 13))
 (segment (start 189.9375 65.5625) (end 189.9375 66.5) (width 0.2) (layer "F.Cu") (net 13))
 (via (at 190 65.5) (size 0.6) (drill 0.3) (layers "F.Cu" "B.Cu") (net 13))
 (via (at 189 70) (size 0.6) (drill 0.3) (layers "F.Cu" "B.Cu") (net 13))
 (segment (start 190 69) (end 190 65.5) (width 0.2) (layer "B.Cu") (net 13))
 (segment (start 189 70) (end 190 69) (width 0.2) (layer "B.Cu") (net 13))
 (segment (start 162.214365 109.5) (end 170.65 109.5) (width 0.2) (layer "F.Cu") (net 22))
 (segment (start 170.65 109.5) (end 171.78 110.63) (width 0.2) (layer "F.Cu") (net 22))
 (segment (start 160.555635 111.73) (end 161.5 110.785635) (width 0.2) (layer "F.Cu") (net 22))
 (segment (start 159.33 111.73) (end 160.555635 111.73) (width 0.2) (layer "F.Cu") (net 22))
 (segment (start 161.5 110.214365) (end 162.214365 109.5) (width 0.2) (layer "F.Cu") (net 22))
 (segment (start 158.66 111.06) (end 159.33 111.73) (width 0.2) (layer "F.Cu") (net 22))
 (segment (start 158.66 88.4555) (end 158.66 111.06) (width 0.2) (layer "F.Cu") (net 22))
 (segment (start 161.5 110.785635) (end 161.5 110.214365) (width 0.2) (layer "F.Cu") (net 22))
 (segment (start 154.2895 84.085) (end 158.66 88.4555) (width 0.2) (layer "F.Cu") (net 22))
 (segment (start 166.22 112.13) (end 167.72 110.63) (width 0.2) (layer "F.Cu") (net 23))
 (segment (start 151 111.5) (end 151.63 112.13) (width 0.2) (layer "F.Cu") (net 23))
 (segment (start 151.63 112.13) (end 166.22 112.13) (width 0.2) (layer "F.Cu") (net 23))
 (segment (start 150.5995 109.733865) (end 150.5995 85.235) (width 0.2) (layer "F.Cu") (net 23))
 (segment (start 151.04 110.174365) (end 150.5995 109.733865) (width 0.2) (layer "F.Cu") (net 23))
 (segment (start 151 111.5) (end 151.04 111.46) (width 0.2) (layer "F.Cu") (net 23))
 (segment (start 150.5995 85.235) (end 151.7495 84.085) (width 0.2) (layer "F.Cu") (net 23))
 (segment (start 151.04 111.46) (end 151.04 110.174365) (width 0.2) (layer "F.Cu") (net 23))
 (segment (start 153.1395 108.7495) (end 153.1395 82.695) (width 0.2) (layer "F.Cu") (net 28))
 (segment (start 153.1395 82.695) (end 154.2895 81.545) (width 0.2) (layer "F.Cu") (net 28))
 (segment (start 155.02 110.63) (end 153.1395 108.7495) (width 0.2) (layer "F.Cu") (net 28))
 (segment (start 154.765846 80.395) (end 160.1 85.729154) (width 0.2) (layer "F.Cu") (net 26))
 (segment (start 160.1 85.729154) (end 160.1 110.63) (width 0.2) (layer "F.Cu") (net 26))
 (segment (start 151.7495 81.545) (end 152.8995 80.395) (width 0.2) (layer "F.Cu") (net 26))
 (segment (start 152.8995 80.395) (end 154.765846 80.395) (width 0.2) (layer "F.Cu") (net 26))
 (segment (start 187.5 95.4) (end 187.5 98.225) (width 0.2) (layer "F.Cu") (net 42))
 (segment (start 187.5 98.225) (end 187.775 98.5) (width 0.2) (layer "F.Cu") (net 42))
 (segment (start 188 91.5) (end 188 90) (width 0.2) (layer "F.Cu") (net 35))
 (segment (start 188 90) (end 187 89) (width 0.2) (layer "F.Cu") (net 35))
 (segment (start 174.075 85.54) (end 174.075 83.615) (width 0.2) (layer "F.Cu") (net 33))
 (segment (start 174.075 83.615) (end 174 83.54) (width 0.2) (layer "F.Cu") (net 33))
 (segment (start 187.7625 67.15) (end 188.0625 67.45) (width 0.2) (layer "F.Cu") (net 2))
 (segment (start 185.5 67.15) (end 187.7625 67.15) (width 0.2) (layer "F.Cu") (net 2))
 (segment (start 185.5 67.15) (end 183 67) (width 0.2) (layer "F.Cu") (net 2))
 (segment (start 186 91.5) (end 185.85 91.35) (width 0.2) (layer "F.Cu") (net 2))
 (segment (start 185.85 91.35) (end 185.85 71.15) (width 0.2) (layer "F.Cu") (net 2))
 (segment (start 185.85 71.15) (end 186 71) (width 0.2) (layer "F.Cu") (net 2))
 (segment (start 183 67) (end 183.15 67.15) (width 0.2) (layer "F.Cu") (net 2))
 (via (at 186 71) (size 0.6) (drill 0.3) (layers "F.Cu" "B.Cu") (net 2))
 (via (at 183 67) (size 0.6) (drill 0.3) (layers "F.Cu" "B.Cu") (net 2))
 (segment (start 183 67) (end 186 70) (width 0.2) (layer "B.Cu") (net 2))
 (segment (start 186 70) (end 186 71) (width 0.2) (layer "B.Cu") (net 2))
 (segment (start 189 83) (end 189 86) (width 0.2) (layer "F.Cu") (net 32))
 (segment (start 189 86) (end 188.776304 86) (width 0.2) (layer "F.Cu") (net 32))
 (segment (start 186.25 90.79259) (end 186.25 82.471948) (width 0.2) (layer "F.Cu") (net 32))
 (segment (start 186.759448 81.9625) (end 187.440552 81.9625) (width 0.2) (layer "F.Cu") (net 32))
 (segment (start 186.25 82.471948) (end 186.759448 81.9625) (width 0.2) (layer "F.Cu") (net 32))
 (segment (start 186.5 91.04259) (end 186.25 90.79259) (width 0.2) (layer "F.Cu") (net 32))
 (segment (start 187.440552 81.9625) (end 189 83.521948) (width 0.2) (layer "F.Cu") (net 32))
 (segment (start 189 83.521948) (end 189 86) (width 0.2) (layer "F.Cu") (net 32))
 (segment (start 186.5 91.5) (end 186.5 91.04259) (width 0.2) (layer "F.Cu") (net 32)))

